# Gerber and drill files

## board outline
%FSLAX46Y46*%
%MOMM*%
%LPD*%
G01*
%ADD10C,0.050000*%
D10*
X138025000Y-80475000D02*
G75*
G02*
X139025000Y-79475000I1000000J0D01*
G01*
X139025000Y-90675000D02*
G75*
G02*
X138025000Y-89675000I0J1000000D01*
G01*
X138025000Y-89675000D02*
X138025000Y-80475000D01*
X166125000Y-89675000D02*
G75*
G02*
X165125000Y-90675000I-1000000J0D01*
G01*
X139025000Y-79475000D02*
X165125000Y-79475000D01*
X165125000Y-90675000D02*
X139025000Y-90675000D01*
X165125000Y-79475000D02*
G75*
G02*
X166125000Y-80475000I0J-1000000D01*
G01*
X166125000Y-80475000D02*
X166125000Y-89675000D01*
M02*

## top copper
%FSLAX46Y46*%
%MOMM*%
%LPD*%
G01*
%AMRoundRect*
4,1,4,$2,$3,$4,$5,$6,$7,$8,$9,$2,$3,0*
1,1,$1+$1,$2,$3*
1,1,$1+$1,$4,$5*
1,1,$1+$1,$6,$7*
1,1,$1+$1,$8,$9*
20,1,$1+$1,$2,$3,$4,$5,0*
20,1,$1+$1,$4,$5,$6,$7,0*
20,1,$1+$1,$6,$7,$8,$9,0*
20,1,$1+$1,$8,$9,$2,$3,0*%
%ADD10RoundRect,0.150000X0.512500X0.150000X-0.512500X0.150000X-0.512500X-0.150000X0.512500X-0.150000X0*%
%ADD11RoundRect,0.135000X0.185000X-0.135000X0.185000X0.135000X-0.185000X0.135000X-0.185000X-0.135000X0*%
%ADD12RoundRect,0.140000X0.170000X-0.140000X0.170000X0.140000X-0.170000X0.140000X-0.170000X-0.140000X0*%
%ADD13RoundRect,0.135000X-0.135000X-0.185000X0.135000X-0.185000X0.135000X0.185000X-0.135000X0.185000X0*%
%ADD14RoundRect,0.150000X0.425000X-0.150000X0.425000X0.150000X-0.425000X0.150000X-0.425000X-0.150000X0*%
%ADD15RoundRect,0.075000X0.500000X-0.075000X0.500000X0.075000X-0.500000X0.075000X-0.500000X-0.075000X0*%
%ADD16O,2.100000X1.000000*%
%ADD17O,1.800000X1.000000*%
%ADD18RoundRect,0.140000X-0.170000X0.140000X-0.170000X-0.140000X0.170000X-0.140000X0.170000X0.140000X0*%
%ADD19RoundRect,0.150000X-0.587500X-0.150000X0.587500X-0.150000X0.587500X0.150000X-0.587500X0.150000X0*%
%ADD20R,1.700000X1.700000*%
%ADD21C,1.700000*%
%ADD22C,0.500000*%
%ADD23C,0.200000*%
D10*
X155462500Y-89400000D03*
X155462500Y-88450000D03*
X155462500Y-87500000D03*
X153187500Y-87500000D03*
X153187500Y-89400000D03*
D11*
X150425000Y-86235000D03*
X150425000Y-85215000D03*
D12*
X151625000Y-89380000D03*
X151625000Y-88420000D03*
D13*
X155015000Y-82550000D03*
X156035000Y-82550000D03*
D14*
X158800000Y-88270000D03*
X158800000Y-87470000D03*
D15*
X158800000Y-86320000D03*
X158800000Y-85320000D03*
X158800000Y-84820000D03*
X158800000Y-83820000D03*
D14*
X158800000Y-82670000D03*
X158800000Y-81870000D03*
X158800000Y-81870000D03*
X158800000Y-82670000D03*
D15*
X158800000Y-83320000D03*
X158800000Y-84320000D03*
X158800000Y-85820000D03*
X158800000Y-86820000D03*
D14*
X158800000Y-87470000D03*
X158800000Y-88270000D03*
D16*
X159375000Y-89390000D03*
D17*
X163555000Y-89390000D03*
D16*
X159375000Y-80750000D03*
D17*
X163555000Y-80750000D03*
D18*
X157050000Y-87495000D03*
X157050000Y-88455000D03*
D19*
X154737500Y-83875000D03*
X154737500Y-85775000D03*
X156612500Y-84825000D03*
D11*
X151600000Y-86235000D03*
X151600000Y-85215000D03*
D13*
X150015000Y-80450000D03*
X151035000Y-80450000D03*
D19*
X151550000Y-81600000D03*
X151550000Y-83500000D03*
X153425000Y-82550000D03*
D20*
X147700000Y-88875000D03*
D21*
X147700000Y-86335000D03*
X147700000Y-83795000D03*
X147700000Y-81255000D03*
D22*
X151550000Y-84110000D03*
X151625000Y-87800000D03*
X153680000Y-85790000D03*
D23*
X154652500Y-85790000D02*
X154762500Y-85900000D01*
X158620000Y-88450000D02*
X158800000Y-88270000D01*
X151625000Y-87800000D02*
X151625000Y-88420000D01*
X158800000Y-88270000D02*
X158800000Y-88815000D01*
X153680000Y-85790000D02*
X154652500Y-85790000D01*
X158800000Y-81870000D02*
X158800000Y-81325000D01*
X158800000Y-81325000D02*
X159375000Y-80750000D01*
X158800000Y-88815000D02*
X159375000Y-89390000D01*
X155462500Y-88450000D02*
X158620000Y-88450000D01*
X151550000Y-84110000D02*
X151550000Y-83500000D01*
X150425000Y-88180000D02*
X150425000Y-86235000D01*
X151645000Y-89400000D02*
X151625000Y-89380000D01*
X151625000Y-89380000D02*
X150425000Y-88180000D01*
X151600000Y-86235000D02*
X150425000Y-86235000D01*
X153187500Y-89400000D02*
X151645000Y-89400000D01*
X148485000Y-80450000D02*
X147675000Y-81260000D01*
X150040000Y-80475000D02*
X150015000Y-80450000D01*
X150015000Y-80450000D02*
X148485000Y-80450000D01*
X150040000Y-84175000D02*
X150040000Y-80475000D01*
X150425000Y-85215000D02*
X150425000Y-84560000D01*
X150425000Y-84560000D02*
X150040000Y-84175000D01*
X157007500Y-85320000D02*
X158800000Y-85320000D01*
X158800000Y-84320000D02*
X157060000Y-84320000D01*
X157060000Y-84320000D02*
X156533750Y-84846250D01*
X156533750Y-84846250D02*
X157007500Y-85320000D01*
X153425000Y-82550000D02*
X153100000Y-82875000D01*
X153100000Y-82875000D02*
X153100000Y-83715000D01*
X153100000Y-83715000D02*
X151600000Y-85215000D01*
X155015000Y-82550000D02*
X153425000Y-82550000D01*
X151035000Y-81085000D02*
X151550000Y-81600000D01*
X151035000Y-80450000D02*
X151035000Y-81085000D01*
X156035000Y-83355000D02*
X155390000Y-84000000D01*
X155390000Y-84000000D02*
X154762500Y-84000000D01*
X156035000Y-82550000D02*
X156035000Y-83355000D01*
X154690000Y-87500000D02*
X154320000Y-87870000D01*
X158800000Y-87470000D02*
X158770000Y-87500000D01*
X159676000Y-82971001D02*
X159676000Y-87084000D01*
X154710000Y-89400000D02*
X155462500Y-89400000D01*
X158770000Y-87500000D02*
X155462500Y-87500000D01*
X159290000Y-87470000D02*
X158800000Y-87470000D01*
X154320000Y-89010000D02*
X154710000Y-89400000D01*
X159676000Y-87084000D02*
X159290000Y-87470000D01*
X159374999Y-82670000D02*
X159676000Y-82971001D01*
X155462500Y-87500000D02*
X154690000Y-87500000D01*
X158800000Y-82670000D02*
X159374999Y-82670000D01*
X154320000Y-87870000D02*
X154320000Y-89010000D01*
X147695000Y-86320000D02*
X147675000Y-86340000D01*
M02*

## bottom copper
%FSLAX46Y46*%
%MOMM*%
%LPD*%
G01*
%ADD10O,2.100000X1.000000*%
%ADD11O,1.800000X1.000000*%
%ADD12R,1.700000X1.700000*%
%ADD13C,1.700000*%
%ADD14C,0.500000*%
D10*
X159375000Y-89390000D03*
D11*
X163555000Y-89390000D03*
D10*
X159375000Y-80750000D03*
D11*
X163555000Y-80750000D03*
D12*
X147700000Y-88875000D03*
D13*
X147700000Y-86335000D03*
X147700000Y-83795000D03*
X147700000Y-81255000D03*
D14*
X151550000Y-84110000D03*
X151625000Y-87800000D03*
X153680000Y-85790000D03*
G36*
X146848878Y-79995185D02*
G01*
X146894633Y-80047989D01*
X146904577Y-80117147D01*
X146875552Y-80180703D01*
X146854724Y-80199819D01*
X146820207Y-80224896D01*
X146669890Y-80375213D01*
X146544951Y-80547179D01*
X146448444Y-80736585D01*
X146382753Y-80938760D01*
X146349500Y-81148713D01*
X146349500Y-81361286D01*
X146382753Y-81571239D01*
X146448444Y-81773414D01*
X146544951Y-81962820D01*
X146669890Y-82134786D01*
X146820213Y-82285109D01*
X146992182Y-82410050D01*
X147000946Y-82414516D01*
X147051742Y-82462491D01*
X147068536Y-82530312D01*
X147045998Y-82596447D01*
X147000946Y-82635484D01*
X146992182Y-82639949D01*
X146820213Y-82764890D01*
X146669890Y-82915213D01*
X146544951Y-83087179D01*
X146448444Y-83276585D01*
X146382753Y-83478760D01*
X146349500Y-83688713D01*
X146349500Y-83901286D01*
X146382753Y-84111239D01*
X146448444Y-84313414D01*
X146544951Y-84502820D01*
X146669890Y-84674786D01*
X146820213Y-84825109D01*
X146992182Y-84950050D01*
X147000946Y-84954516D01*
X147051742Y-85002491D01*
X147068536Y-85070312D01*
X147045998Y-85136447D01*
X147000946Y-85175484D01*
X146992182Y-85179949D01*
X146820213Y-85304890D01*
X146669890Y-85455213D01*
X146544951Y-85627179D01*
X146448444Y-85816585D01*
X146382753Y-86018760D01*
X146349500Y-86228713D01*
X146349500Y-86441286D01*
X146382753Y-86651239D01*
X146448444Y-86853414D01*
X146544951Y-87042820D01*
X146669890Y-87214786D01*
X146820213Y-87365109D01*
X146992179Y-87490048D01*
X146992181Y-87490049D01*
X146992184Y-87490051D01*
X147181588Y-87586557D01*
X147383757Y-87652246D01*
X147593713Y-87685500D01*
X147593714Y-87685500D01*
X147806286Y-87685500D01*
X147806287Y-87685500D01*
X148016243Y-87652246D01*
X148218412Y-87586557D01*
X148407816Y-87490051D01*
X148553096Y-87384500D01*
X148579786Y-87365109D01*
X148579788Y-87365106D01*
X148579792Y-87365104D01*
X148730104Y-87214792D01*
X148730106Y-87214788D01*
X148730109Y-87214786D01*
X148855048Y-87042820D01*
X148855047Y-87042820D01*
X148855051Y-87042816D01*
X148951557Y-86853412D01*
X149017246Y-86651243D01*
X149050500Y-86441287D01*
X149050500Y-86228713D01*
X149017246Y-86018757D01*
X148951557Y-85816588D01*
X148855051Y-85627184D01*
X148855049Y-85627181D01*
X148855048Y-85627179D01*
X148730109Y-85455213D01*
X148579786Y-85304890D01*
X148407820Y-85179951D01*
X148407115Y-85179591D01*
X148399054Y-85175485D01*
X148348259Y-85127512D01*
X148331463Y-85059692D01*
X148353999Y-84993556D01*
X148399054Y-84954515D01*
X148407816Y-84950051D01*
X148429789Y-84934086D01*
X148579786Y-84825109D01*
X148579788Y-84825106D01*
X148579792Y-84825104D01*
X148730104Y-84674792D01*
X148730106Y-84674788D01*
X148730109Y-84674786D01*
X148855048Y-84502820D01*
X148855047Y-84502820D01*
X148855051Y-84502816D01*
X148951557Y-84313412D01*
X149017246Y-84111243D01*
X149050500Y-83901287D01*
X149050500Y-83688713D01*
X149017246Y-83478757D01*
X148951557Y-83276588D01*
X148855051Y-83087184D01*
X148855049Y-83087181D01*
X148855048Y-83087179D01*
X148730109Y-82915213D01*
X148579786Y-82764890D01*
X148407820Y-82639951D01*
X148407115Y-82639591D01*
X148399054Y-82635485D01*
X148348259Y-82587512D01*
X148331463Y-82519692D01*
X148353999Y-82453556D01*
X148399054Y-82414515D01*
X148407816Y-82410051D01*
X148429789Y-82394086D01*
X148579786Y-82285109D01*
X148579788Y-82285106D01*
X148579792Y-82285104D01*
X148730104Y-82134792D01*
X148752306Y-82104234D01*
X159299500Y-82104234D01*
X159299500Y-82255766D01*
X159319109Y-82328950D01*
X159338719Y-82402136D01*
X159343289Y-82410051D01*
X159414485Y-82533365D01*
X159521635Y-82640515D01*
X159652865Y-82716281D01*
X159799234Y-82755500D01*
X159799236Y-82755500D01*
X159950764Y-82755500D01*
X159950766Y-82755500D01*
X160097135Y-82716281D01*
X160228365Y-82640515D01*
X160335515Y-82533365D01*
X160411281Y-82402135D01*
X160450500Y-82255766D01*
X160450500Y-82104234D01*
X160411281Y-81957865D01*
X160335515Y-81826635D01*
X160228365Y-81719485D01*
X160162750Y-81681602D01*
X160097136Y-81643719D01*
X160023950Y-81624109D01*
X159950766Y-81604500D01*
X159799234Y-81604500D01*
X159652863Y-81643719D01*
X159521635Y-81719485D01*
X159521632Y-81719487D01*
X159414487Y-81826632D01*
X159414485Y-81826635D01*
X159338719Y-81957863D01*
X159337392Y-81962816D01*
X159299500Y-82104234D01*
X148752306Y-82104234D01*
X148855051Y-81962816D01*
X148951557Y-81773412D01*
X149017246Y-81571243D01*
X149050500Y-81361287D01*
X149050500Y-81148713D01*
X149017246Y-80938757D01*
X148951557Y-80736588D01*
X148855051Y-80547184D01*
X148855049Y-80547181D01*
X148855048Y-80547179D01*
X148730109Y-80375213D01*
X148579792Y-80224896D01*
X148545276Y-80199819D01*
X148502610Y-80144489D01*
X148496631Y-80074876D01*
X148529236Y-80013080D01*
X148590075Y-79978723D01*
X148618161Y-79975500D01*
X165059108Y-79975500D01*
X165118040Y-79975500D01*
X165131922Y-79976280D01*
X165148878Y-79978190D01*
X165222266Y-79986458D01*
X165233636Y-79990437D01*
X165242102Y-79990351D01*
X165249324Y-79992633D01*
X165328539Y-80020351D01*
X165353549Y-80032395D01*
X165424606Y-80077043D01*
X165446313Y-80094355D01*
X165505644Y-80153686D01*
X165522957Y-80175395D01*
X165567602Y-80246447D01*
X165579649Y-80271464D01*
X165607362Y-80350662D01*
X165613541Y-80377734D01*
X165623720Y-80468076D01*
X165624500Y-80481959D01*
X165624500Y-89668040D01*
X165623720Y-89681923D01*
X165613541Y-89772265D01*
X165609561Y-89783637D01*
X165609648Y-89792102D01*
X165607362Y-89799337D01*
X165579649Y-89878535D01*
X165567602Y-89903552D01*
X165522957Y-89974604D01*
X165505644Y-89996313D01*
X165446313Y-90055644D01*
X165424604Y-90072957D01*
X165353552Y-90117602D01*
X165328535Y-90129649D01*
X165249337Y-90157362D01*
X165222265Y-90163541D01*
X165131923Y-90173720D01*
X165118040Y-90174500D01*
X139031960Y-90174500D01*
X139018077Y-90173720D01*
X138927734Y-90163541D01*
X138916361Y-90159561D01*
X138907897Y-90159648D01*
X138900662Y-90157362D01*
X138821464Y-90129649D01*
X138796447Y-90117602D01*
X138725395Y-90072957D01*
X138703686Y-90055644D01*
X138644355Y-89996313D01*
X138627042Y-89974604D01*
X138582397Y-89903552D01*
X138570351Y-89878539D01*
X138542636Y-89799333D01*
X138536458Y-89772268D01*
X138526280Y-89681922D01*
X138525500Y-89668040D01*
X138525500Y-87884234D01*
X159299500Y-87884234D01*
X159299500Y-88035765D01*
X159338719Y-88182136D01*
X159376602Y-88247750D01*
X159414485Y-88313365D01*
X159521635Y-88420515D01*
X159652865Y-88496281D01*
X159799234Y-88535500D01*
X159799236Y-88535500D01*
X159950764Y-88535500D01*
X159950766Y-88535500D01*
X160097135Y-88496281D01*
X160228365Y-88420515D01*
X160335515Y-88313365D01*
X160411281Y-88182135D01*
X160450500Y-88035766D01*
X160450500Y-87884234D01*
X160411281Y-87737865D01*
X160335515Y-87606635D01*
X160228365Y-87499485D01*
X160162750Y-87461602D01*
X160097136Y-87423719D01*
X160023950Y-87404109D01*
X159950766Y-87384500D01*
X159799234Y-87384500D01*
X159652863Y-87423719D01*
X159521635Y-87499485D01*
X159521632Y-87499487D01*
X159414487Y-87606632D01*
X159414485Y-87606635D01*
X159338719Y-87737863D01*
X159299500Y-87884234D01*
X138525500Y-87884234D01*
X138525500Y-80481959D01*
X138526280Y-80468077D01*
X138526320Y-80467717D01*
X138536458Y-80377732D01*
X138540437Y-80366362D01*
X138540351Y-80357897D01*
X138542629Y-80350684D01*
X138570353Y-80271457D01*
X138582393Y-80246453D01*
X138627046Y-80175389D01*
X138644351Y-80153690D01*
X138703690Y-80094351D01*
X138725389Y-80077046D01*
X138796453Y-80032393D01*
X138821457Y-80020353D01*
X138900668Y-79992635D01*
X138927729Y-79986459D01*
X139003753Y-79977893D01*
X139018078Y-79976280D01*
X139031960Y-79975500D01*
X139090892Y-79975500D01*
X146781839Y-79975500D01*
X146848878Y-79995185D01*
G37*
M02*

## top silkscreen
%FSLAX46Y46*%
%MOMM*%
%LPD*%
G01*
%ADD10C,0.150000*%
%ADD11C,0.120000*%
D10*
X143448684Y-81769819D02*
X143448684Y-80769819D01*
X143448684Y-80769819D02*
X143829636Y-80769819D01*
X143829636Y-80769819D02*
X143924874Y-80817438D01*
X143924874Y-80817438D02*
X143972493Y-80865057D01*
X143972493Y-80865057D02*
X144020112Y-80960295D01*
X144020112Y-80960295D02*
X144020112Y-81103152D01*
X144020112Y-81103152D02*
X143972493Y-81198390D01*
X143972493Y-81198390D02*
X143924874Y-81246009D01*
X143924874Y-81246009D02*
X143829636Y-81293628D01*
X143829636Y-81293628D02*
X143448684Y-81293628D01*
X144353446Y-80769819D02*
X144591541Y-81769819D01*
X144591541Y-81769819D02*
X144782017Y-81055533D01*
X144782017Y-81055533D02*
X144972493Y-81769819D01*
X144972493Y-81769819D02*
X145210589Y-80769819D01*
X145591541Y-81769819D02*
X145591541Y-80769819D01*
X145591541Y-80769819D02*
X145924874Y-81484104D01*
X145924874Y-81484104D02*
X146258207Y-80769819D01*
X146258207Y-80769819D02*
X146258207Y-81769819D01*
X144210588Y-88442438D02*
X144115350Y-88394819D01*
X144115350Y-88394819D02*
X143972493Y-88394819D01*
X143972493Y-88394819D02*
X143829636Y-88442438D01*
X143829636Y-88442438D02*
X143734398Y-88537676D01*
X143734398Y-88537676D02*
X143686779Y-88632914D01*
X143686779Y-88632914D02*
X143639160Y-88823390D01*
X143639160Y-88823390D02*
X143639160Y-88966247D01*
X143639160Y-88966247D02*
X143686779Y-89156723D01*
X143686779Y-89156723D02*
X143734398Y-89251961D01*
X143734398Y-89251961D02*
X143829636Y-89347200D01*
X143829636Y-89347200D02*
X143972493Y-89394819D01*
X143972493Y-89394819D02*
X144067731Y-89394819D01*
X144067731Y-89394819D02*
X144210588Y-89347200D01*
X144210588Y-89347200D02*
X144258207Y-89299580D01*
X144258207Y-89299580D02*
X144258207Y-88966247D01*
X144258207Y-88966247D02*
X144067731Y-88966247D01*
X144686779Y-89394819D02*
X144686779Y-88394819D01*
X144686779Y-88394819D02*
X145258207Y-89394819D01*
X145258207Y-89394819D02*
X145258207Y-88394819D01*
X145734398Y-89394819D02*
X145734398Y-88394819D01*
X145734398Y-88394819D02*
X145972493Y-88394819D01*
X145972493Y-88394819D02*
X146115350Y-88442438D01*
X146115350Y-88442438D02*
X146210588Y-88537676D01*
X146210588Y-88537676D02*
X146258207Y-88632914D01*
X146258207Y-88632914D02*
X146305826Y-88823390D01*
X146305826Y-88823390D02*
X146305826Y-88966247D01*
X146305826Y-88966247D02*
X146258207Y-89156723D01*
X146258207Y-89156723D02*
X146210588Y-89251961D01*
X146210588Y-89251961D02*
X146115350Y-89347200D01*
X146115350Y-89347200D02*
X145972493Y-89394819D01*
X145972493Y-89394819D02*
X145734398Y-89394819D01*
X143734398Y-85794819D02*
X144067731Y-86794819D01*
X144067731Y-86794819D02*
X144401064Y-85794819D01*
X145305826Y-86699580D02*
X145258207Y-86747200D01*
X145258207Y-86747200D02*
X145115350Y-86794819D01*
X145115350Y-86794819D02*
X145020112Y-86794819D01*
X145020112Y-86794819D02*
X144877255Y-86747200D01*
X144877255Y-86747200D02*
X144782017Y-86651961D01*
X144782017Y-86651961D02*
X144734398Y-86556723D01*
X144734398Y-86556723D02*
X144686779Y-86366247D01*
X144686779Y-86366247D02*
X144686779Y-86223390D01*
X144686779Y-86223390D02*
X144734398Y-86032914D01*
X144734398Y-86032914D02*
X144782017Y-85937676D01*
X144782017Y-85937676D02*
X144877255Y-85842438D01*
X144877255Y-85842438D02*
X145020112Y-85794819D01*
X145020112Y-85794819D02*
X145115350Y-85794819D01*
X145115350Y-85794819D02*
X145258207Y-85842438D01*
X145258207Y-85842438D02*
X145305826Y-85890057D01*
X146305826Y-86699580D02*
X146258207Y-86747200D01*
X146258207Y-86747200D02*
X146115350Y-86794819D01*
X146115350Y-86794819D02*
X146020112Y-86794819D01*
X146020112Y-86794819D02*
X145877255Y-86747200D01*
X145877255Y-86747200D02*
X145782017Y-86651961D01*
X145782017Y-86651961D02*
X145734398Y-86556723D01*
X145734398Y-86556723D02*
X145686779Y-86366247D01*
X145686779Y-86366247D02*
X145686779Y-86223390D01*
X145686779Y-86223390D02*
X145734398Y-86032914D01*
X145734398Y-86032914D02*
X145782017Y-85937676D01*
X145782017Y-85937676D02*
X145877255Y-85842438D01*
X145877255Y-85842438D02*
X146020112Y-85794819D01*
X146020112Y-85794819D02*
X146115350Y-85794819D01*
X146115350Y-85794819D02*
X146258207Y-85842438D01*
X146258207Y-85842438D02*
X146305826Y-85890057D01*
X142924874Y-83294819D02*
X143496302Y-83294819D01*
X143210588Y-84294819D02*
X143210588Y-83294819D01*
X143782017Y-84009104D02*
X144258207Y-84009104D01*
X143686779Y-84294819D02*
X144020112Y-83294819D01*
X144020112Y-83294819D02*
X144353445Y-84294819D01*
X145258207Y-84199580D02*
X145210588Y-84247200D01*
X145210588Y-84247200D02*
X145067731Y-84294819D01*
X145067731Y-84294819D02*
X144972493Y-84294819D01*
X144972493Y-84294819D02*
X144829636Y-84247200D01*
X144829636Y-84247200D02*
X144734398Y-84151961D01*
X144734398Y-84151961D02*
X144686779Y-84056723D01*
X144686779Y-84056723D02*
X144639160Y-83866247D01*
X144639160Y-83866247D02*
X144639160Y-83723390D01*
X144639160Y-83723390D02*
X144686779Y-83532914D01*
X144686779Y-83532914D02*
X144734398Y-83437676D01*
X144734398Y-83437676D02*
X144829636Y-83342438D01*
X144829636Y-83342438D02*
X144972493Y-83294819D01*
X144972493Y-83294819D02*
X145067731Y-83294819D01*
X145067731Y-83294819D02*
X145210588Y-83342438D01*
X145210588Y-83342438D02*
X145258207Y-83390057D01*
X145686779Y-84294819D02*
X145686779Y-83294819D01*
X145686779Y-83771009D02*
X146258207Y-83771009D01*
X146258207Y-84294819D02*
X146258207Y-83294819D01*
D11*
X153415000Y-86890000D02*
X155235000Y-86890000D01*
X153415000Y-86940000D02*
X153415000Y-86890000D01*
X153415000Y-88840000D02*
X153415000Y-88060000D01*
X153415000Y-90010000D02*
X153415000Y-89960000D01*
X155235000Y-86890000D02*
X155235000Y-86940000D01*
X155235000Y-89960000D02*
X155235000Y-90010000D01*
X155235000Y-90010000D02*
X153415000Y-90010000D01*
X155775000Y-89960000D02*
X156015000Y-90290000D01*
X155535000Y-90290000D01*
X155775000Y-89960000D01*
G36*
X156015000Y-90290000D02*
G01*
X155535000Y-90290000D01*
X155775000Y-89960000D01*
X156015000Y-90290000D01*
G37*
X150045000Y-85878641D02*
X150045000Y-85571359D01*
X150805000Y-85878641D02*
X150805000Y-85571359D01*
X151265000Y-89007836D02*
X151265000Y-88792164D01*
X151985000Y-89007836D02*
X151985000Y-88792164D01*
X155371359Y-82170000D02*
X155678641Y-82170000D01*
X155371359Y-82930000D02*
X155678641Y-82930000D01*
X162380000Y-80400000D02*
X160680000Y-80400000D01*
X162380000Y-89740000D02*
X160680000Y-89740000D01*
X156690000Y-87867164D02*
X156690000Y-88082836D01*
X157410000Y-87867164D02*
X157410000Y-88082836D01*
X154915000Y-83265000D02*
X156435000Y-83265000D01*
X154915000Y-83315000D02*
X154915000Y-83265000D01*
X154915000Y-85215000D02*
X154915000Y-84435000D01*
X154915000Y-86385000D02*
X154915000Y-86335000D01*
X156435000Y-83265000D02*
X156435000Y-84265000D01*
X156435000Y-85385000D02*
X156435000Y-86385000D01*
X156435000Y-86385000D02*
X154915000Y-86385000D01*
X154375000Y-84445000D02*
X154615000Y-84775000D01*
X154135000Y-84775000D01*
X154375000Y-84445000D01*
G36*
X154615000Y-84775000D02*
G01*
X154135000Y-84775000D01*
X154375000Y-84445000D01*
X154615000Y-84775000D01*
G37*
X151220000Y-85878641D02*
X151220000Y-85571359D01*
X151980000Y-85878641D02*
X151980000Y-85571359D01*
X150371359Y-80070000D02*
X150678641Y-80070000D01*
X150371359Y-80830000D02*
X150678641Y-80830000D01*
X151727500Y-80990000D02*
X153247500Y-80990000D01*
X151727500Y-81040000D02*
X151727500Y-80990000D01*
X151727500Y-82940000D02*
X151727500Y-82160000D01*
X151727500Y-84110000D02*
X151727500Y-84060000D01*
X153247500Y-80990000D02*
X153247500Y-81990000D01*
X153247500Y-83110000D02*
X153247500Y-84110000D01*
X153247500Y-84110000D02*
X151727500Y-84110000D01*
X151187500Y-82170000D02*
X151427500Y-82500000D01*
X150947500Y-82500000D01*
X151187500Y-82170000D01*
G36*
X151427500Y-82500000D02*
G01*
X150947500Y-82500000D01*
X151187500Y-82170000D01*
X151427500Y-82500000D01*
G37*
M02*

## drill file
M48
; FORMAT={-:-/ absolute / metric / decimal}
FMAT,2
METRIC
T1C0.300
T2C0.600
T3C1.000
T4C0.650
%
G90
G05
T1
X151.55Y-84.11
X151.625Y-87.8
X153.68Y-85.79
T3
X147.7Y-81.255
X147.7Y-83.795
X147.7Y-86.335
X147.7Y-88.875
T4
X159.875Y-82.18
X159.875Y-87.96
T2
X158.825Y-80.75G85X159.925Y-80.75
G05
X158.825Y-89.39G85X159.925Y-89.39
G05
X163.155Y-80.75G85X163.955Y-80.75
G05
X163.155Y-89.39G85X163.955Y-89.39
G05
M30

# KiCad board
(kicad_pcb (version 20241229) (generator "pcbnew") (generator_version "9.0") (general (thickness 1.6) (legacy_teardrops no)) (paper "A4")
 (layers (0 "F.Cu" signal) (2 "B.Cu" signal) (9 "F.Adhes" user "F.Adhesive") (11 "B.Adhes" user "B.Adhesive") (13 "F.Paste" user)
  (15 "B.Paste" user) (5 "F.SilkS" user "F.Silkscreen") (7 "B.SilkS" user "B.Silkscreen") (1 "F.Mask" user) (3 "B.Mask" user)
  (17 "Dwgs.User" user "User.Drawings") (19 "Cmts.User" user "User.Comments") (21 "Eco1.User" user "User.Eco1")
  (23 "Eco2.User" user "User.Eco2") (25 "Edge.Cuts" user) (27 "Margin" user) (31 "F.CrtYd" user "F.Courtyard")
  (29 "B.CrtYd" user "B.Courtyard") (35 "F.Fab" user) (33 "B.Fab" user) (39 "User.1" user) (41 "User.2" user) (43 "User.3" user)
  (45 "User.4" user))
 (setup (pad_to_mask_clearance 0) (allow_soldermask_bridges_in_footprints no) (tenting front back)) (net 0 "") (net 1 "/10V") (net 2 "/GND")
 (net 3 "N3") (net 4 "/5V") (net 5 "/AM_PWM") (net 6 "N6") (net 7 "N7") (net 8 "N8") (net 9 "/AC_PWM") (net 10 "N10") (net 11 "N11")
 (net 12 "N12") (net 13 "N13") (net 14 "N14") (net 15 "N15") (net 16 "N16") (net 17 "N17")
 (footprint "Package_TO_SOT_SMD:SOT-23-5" (layer "F.Cu") (at 154.325 88.45 180)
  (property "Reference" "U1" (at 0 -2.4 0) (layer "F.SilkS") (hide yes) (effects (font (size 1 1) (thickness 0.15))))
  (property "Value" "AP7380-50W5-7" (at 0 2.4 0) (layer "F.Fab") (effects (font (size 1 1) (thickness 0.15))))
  (fp_line (start 0.91 1.56) (end -0.91 1.56) (stroke (width 0.12) (type solid)) (layer "F.SilkS"))
  (fp_line (start 0.91 1.51) (end 0.91 1.56) (stroke (width 0.12) (type solid)) (layer "F.SilkS"))
  (fp_line (start 0.91 -0.39) (end 0.91 0.39) (stroke (width 0.12) (type solid)) (layer "F.SilkS"))
  (fp_line (start 0.91 -1.56) (end 0.91 -1.51) (stroke (width 0.12) (type solid)) (layer "F.SilkS"))
  (fp_line (start -0.91 1.56) (end -0.91 1.51) (stroke (width 0.12) (type solid)) (layer "F.SilkS"))
  (fp_line (start -0.91 -1.51) (end -0.91 -1.56) (stroke (width 0.12) (type solid)) (layer "F.SilkS"))
  (fp_line (start -0.91 -1.56) (end 0.91 -1.56) (stroke (width 0.12) (type solid)) (layer "F.SilkS"))
  (fp_poly (pts (xy -1.45 -1.51) (xy -1.69 -1.84) (xy -1.21 -1.84)) (stroke (width 0.12) (type solid)) (fill yes) (layer "F.SilkS"))
  (pad "1" smd roundrect (at -1.1375 -0.95 180) (size 1.325 0.6) (layers "F.Cu" "F.Mask" "F.Paste") (roundrect_rratio 0.25) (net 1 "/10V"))
  (pad "2" smd roundrect (at -1.1375 0 180) (size 1.325 0.6) (layers "F.Cu" "F.Mask" "F.Paste") (roundrect_rratio 0.25) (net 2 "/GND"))
  (pad "3" smd roundrect (at -1.1375 0.95 180) (size 1.325 0.6) (layers "F.Cu" "F.Mask" "F.Paste") (roundrect_rratio 0.25) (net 1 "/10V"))
  (pad "4" smd roundrect (at 1.1375 0.95 180) (size 1.325 0.6) (layers "F.Cu" "F.Mask" "F.Paste") (roundrect_rratio 0.25) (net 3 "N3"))
  (pad "5" smd roundrect (at 1.1375 -0.95 180) (size 1.325 0.6) (layers "F.Cu" "F.Mask" "F.Paste") (roundrect_rratio 0.25) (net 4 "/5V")))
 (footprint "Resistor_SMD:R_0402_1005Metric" (layer "F.Cu") (at 150.425 85.725 90)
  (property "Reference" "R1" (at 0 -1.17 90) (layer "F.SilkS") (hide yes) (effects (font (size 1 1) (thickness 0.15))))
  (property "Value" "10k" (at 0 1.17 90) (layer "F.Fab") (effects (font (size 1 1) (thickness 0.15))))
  (fp_line (start -0.153641 -0.38) (end 0.153641 -0.38) (stroke (width 0.12) (type solid)) (layer "F.SilkS"))
  (fp_line (start -0.153641 0.38) (end 0.153641 0.38) (stroke (width 0.12) (type solid)) (layer "F.SilkS"))
  (pad "1" smd roundrect (at -0.51 0 90) (size 0.54 0.64) (layers "F.Cu" "F.Mask" "F.Paste") (roundrect_rratio 0.25) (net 4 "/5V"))
  (pad "2" smd roundrect (at 0.51 0 90) (size 0.54 0.64) (layers "F.Cu" "F.Mask" "F.Paste") (roundrect_rratio 0.25) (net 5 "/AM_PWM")))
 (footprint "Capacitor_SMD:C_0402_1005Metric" (layer "F.Cu") (at 151.625 88.9 90)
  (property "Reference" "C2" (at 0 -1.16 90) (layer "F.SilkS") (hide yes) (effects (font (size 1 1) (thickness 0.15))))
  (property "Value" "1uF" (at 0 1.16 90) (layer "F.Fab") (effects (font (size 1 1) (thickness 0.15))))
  (fp_line (start -0.107836 -0.36) (end 0.107836 -0.36) (stroke (width 0.12) (type solid)) (layer "F.SilkS"))
  (fp_line (start -0.107836 0.36) (end 0.107836 0.36) (stroke (width 0.12) (type solid)) (layer "F.SilkS"))
  (pad "1" smd roundrect (at -0.48 0 90) (size 0.56 0.62) (layers "F.Cu" "F.Mask" "F.Paste") (roundrect_rratio 0.25) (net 4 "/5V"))
  (pad "2" smd roundrect (at 0.48 0 90) (size 0.56 0.62) (layers "F.Cu" "F.Mask" "F.Paste") (roundrect_rratio 0.25) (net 2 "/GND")))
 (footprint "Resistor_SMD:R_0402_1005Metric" (layer "F.Cu") (at 155.525 82.55)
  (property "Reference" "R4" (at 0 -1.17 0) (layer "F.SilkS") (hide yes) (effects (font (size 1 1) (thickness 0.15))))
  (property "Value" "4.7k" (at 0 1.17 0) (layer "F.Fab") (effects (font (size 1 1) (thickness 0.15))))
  (fp_line (start -0.153641 -0.38) (end 0.153641 -0.38) (stroke (width 0.12) (type solid)) (layer "F.SilkS"))
  (fp_line (start -0.153641 0.38) (end 0.153641 0.38) (stroke (width 0.12) (type solid)) (layer "F.SilkS"))
  (pad "1" smd roundrect (at -0.51 0) (size 0.54 0.64) (layers "F.Cu" "F.Mask" "F.Paste") (roundrect_rratio 0.25) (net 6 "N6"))
  (pad "2" smd roundrect (at 0.51 0) (size 0.54 0.64) (layers "F.Cu" "F.Mask" "F.Paste") (roundrect_rratio 0.25) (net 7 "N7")))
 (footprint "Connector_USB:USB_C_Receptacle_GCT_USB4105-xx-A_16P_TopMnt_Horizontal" (layer "F.Cu") (at 162.48 85.07 90)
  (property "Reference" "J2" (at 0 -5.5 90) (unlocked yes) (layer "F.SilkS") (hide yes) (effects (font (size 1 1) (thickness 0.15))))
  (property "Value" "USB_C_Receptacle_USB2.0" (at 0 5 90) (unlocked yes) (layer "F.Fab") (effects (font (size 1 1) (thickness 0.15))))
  (fp_line (start 4.67 -0.1) (end 4.67 -1.8) (stroke (width 0.12) (type solid)) (layer "F.SilkS"))
  (fp_line (start -4.67 -0.1) (end -4.67 -1.8) (stroke (width 0.12) (type solid)) (layer "F.SilkS"))
  (pad "" np_thru_hole circle (at -2.89 -2.605 90) (size 0.65 0.65) (drill 0.65) (layers "*.Cu" "*.Mask"))
  (pad "" np_thru_hole circle (at 2.89 -2.605 90) (size 0.65 0.65) (drill 0.65) (layers "*.Cu" "*.Mask"))
  (pad "A1" smd roundrect (at -3.2 -3.68 90) (size 0.6 1.15) (layers "F.Cu" "F.Mask" "F.Paste") (roundrect_rratio 0.25) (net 2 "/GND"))
  (pad "A4" smd roundrect (at -2.4 -3.68 90) (size 0.6 1.15) (layers "F.Cu" "F.Mask" "F.Paste") (roundrect_rratio 0.25) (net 1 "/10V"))
  (pad "A5" smd roundrect (at -1.25 -3.68 90) (size 0.3 1.15) (layers "F.Cu" "F.Mask" "F.Paste") (roundrect_rratio 0.25) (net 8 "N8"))
  (pad "A6" smd roundrect (at -0.25 -3.68 90) (size 0.3 1.15) (layers "F.Cu" "F.Mask" "F.Paste") (roundrect_rratio 0.25) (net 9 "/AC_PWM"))
  (pad "A7" smd roundrect (at 0.25 -3.68 90) (size 0.3 1.15) (layers "F.Cu" "F.Mask" "F.Paste") (roundrect_rratio 0.25) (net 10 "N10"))
  (pad "A8" smd roundrect (at 1.25 -3.68 90) (size 0.3 1.15) (layers "F.Cu" "F.Mask" "F.Paste") (roundrect_rratio 0.25) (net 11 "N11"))
  (pad "A9" smd roundrect (at 2.4 -3.68 90) (size 0.6 1.15) (layers "F.Cu" "F.Mask" "F.Paste") (roundrect_rratio 0.25) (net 1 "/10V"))
  (pad "A12" smd roundrect (at 3.2 -3.68 90) (size 0.6 1.15) (layers "F.Cu" "F.Mask" "F.Paste") (roundrect_rratio 0.25) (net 2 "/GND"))
  (pad "B1" smd roundrect (at 3.2 -3.68 90) (size 0.6 1.15) (layers "F.Cu" "F.Mask" "F.Paste") (roundrect_rratio 0.25) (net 2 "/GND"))
  (pad "B4" smd roundrect (at 2.4 -3.68 90) (size 0.6 1.15) (layers "F.Cu" "F.Mask" "F.Paste") (roundrect_rratio 0.25) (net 1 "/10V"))
  (pad "B5" smd roundrect (at 1.75 -3.68 90) (size 0.3 1.15) (layers "F.Cu" "F.Mask" "F.Paste") (roundrect_rratio 0.25) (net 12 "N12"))
  (pad "B6" smd roundrect (at 0.75 -3.68 90) (size 0.3 1.15) (layers "F.Cu" "F.Mask" "F.Paste") (roundrect_rratio 0.25) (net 9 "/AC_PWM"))
  (pad "B7" smd roundrect (at -0.75 -3.68 90) (size 0.3 1.15) (layers "F.Cu" "F.Mask" "F.Paste") (roundrect_rratio 0.25) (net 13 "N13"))
  (pad "B8" smd roundrect (at -1.75 -3.68 90) (size 0.3 1.15) (layers "F.Cu" "F.Mask" "F.Paste") (roundrect_rratio 0.25) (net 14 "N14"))
  (pad "B9" smd roundrect (at -2.4 -3.68 90) (size 0.6 1.15) (layers "F.Cu" "F.Mask" "F.Paste") (roundrect_rratio 0.25) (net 1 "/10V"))
  (pad "B12" smd roundrect (at -3.2 -3.68 90) (size 0.6 1.15) (layers "F.Cu" "F.Mask" "F.Paste") (roundrect_rratio 0.25) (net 2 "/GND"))
  (pad "S1" thru_hole oval (at -4.32 -3.105 90) (size 1 2.1) (drill oval 0.6 1.7) (layers "*.Cu" "*.Mask" "F.Paste")
   (remove_unused_layers no) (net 2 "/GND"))
  (pad "S1" thru_hole oval (at -4.32 1.075 90) (size 1 1.8) (drill oval 0.6 1.4) (layers "*.Cu" "*.Mask" "F.Paste")
   (remove_unused_layers no) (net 2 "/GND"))
  (pad "S1" thru_hole oval (at 4.32 -3.105 90) (size 1 2.1) (drill oval 0.6 1.7) (layers "*.Cu" "*.Mask" "F.Paste")
   (remove_unused_layers yes) (keep_end_layers yes) (zone_layer_connections) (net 2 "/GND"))
  (pad "S1" thru_hole oval (at 4.32 1.075 90) (size 1 1.8) (drill oval 0.6 1.4) (layers "*.Cu" "*.Mask" "F.Paste") (remove_unused_layers no)
   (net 2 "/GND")))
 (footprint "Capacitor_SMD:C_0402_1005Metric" (layer "F.Cu") (at 157.05 87.975 -90)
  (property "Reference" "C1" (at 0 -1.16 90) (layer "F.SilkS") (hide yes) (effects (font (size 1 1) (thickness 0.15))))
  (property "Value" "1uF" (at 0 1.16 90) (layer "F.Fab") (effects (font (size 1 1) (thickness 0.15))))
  (fp_line (start -0.107836 0.36) (end 0.107836 0.36) (stroke (width 0.12) (type solid)) (layer "F.SilkS"))
  (fp_line (start -0.107836 -0.36) (end 0.107836 -0.36) (stroke (width 0.12) (type solid)) (layer "F.SilkS"))
  (pad "1" smd roundrect (at -0.48 0 270) (size 0.56 0.62) (layers "F.Cu" "F.Mask" "F.Paste") (roundrect_rratio 0.25) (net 1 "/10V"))
  (pad "2" smd roundrect (at 0.48 0 270) (size 0.56 0.62) (layers "F.Cu" "F.Mask" "F.Paste") (roundrect_rratio 0.25) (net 2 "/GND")))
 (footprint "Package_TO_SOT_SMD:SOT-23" (layer "F.Cu") (at 155.675 84.825)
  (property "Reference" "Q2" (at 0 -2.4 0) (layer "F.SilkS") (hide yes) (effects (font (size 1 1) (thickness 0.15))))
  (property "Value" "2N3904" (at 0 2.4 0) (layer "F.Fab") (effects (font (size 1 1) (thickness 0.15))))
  (fp_line (start -0.76 -1.56) (end 0.76 -1.56) (stroke (width 0.12) (type solid)) (layer "F.SilkS"))
  (fp_line (start -0.76 -1.51) (end -0.76 -1.56) (stroke (width 0.12) (type solid)) (layer "F.SilkS"))
  (fp_line (start -0.76 0.39) (end -0.76 -0.39) (stroke (width 0.12) (type solid)) (layer "F.SilkS"))
  (fp_line (start -0.76 1.56) (end -0.76 1.51) (stroke (width 0.12) (type solid)) (layer "F.SilkS"))
  (fp_line (start 0.76 -1.56) (end 0.76 -0.56) (stroke (width 0.12) (type solid)) (layer "F.SilkS"))
  (fp_line (start 0.76 0.56) (end 0.76 1.56) (stroke (width 0.12) (type solid)) (layer "F.SilkS"))
  (fp_line (start 0.76 1.56) (end -0.76 1.56) (stroke (width 0.12) (type solid)) (layer "F.SilkS"))
  (fp_poly (pts (xy -1.3 -0.38) (xy -1.06 -0.05) (xy -1.54 -0.05)) (stroke (width 0.12) (type solid)) (fill yes) (layer "F.SilkS"))
  (pad "1" smd roundrect (at -0.9375 -0.95) (size 1.475 0.6) (layers "F.Cu" "F.Mask" "F.Paste") (roundrect_rratio 0.25) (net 7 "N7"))
  (pad "2" smd roundrect (at -0.9375 0.95) (size 1.475 0.6) (layers "F.Cu" "F.Mask" "F.Paste") (roundrect_rratio 0.25) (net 2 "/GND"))
  (pad "3" smd roundrect (at 0.9375 0) (size 1.475 0.6) (layers "F.Cu" "F.Mask" "F.Paste") (roundrect_rratio 0.25) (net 9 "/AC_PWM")))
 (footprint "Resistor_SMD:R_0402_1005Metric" (layer "F.Cu") (at 151.6 85.725 90)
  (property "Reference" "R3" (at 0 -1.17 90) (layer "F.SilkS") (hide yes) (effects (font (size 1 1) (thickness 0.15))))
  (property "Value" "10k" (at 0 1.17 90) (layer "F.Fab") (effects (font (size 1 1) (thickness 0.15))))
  (fp_line (start -0.153641 -0.38) (end 0.153641 -0.38) (stroke (width 0.12) (type solid)) (layer "F.SilkS"))
  (fp_line (start -0.153641 0.38) (end 0.153641 0.38) (stroke (width 0.12) (type solid)) (layer "F.SilkS"))
  (pad "1" smd roundrect (at -0.51 0 90) (size 0.54 0.64) (layers "F.Cu" "F.Mask" "F.Paste") (roundrect_rratio 0.25) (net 4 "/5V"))
  (pad "2" smd roundrect (at 0.51 0 90) (size 0.54 0.64) (layers "F.Cu" "F.Mask" "F.Paste") (roundrect_rratio 0.25) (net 6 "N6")))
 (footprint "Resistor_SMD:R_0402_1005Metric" (layer "F.Cu") (at 150.525 80.45)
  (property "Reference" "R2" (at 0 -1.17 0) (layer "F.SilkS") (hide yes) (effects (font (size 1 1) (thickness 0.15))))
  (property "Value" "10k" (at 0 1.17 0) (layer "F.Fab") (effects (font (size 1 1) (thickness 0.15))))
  (fp_line (start -0.153641 -0.38) (end 0.153641 -0.38) (stroke (width 0.12) (type solid)) (layer "F.SilkS"))
  (fp_line (start -0.153641 0.38) (end 0.153641 0.38) (stroke (width 0.12) (type solid)) (layer "F.SilkS"))
  (pad "1" smd roundrect (at -0.51 0) (size 0.54 0.64) (layers "F.Cu" "F.Mask" "F.Paste") (roundrect_rratio 0.25) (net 5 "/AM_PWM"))
  (pad "2" smd roundrect (at 0.51 0) (size 0.54 0.64) (layers "F.Cu" "F.Mask" "F.Paste") (roundrect_rratio 0.25) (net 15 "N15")))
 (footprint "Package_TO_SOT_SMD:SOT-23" (layer "F.Cu") (at 152.4875 82.55)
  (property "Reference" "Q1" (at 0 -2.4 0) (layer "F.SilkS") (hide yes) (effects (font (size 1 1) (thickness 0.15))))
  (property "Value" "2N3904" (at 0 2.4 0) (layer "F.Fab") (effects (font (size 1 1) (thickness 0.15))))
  (fp_line (start -0.76 -1.56) (end 0.76 -1.56) (stroke (width 0.12) (type solid)) (layer "F.SilkS"))
  (fp_line (start -0.76 -1.51) (end -0.76 -1.56) (stroke (width 0.12) (type solid)) (layer "F.SilkS"))
  (fp_line (start -0.76 0.39) (end -0.76 -0.39) (stroke (width 0.12) (type solid)) (layer "F.SilkS"))
  (fp_line (start -0.76 1.56) (end -0.76 1.51) (stroke (width 0.12) (type solid)) (layer "F.SilkS"))
  (fp_line (start 0.76 -1.56) (end 0.76 -0.56) (stroke (width 0.12) (type solid)) (layer "F.SilkS"))
  (fp_line (start 0.76 0.56) (end 0.76 1.56) (stroke (width 0.12) (type solid)) (layer "F.SilkS"))
  (fp_line (start 0.76 1.56) (end -0.76 1.56) (stroke (width 0.12) (type solid)) (layer "F.SilkS"))
  (fp_poly (pts (xy -1.3 -0.38) (xy -1.06 -0.05) (xy -1.54 -0.05)) (stroke (width 0.12) (type solid)) (fill yes) (layer "F.SilkS"))
  (pad "1" smd roundrect (at -0.9375 -0.95) (size 1.475 0.6) (layers "F.Cu" "F.Mask" "F.Paste") (roundrect_rratio 0.25) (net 15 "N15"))
  (pad "2" smd roundrect (at -0.9375 0.95) (size 1.475 0.6) (layers "F.Cu" "F.Mask" "F.Paste") (roundrect_rratio 0.25) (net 2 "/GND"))
  (pad "3" smd roundrect (at 0.9375 0) (size 1.475 0.6) (layers "F.Cu" "F.Mask" "F.Paste") (roundrect_rratio 0.25) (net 6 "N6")))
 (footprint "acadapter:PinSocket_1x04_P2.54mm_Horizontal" (layer "B.Cu") (at 147.7 88.875)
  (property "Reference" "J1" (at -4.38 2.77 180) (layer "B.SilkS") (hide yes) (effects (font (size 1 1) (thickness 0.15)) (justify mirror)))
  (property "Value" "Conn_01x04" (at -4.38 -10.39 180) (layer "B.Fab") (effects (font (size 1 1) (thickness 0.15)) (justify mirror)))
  (pad "1" thru_hole rect (at 0 0) (size 1.7 1.7) (drill 1) (layers "*.Cu" "*.Mask") (remove_unused_layers no) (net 2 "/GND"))
  (pad "2" thru_hole circle (at 0 -2.54) (size 1.7 1.7) (drill 1) (layers "*.Cu" "*.Mask") (remove_unused_layers no) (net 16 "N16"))
  (pad "3" thru_hole circle (at 0 -5.08) (size 1.7 1.7) (drill 1) (layers "*.Cu" "*.Mask") (remove_unused_layers no) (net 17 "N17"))
  (pad "4" thru_hole circle (at 0 -7.62) (size 1.7 1.7) (drill 1) (layers "*.Cu" "*.Mask") (remove_unused_layers no) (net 5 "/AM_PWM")))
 (gr_arc (start 138.025 80.475) (mid 138.317893 79.767893) (end 139.025 79.475) (stroke (width 0.05) (type default)) (layer "Edge.Cuts"))
 (gr_arc (start 139.025 90.675) (mid 138.317893 90.382107) (end 138.025 89.675) (stroke (width 0.05) (type default)) (layer "Edge.Cuts"))
 (gr_line (start 138.025 89.675) (end 138.025 80.475) (stroke (width 0.05) (type default)) (layer "Edge.Cuts"))
 (gr_arc (start 166.125 89.675) (mid 165.832107 90.382107) (end 165.125 90.675) (stroke (width 0.05) (type default)) (layer "Edge.Cuts"))
 (gr_line (start 139.025 79.475) (end 165.125 79.475) (stroke (width 0.05) (type default)) (layer "Edge.Cuts"))
 (gr_line (start 165.125 90.675) (end 139.025 90.675) (stroke (width 0.05) (type default)) (layer "Edge.Cuts"))
 (gr_arc (start 165.125 79.475) (mid 165.832107 79.767893) (end 166.125 80.475) (stroke (width 0.05) (type default)) (layer "Edge.Cuts"))
 (gr_line (start 166.125 80.475) (end 166.125 89.675) (stroke (width 0.05) (type default)) (layer "Edge.Cuts"))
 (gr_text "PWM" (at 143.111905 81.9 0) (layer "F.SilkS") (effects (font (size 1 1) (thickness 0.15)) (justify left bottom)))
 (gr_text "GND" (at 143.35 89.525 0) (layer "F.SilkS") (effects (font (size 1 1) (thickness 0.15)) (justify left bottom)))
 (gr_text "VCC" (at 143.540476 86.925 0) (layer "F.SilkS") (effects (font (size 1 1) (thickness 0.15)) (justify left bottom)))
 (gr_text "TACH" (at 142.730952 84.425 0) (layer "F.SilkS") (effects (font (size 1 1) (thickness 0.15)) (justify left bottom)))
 (segment (start 154.6525 85.79) (end 154.7625 85.9) (width 0.2) (layer "F.Cu") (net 2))
 (segment (start 158.62 88.45) (end 158.8 88.27) (width 0.2) (layer "F.Cu") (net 2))
 (segment (start 151.625 87.8) (end 151.625 88.42) (width 0.2) (layer "F.Cu") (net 2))
 (segment (start 158.8 88.27) (end 158.8 88.815) (width 0.2) (layer "F.Cu") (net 2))
 (segment (start 153.68 85.79) (end 154.6525 85.79) (width 0.2) (layer "F.Cu") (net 2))
 (segment (start 158.8 81.87) (end 158.8 81.325) (width 0.2) (layer "F.Cu") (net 2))
 (segment (start 158.8 81.325) (end 159.375 80.75) (width 0.2) (layer "F.Cu") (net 2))
 (segment (start 158.8 88.815) (end 159.375 89.39) (width 0.2) (layer "F.Cu") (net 2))
 (segment (start 155.4625 88.45) (end 158.62 88.45) (width 0.2) (layer "F.Cu") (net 2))
 (segment (start 151.55 84.11) (end 151.55 83.5) (width 0.2) (layer "F.Cu") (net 2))
 (via (at 151.55 84.11) (size 0.5) (drill 0.3) (layers "F.Cu" "B.Cu") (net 2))
 (via (at 151.625 87.8) (size 0.5) (drill 0.3) (layers "F.Cu" "B.Cu") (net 2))
 (via (at 153.68 85.79) (size 0.5) (drill 0.3) (layers "F.Cu" "B.Cu") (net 2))
 (segment (start 150.425 88.18) (end 150.425 86.235) (width 0.2) (layer "F.Cu") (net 4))
 (segment (start 151.645 89.4) (end 151.625 89.38) (width 0.2) (layer "F.Cu") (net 4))
 (segment (start 151.625 89.38) (end 150.425 88.18) (width 0.2) (layer "F.Cu") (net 4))
 (segment (start 151.6 86.235) (end 150.425 86.235) (width 0.2) (layer "F.Cu") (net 4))
 (segment (start 153.1875 89.4) (end 151.645 89.4) (width 0.2) (layer "F.Cu") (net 4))
 (segment (start 148.485 80.45) (end 147.675 81.26) (width 0.2) (layer "F.Cu") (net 5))
 (segment (start 150.04 80.475) (end 150.015 80.45) (width 0.2) (layer "F.Cu") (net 5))
 (segment (start 150.015 80.45) (end 148.485 80.45) (width 0.2) (layer "F.Cu") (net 5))
 (segment (start 150.04 84.175) (end 150.04 80.475) (width 0.2) (layer "F.Cu") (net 5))
 (segment (start 150.425 85.215) (end 150.425 84.56) (width 0.2) (layer "F.Cu") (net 5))
 (segment (start 150.425 84.56) (end 150.04 84.175) (width 0.2) (layer "F.Cu") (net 5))
 (segment (start 157.0075 85.32) (end 158.8 85.32) (width 0.2) (layer "F.Cu") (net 9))
 (segment (start 158.8 84.32) (end 157.06 84.32) (width 0.2) (layer "F.Cu") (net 9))
 (segment (start 157.06 84.32) (end 156.53375 84.84625) (width 0.2) (layer "F.Cu") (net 9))
 (segment (start 156.53375 84.84625) (end 157.0075 85.32) (width 0.2) (layer "F.Cu") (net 9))
 (segment (start 153.425 82.55) (end 153.1 82.875) (width 0.2) (layer "F.Cu") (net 6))
 (segment (start 153.1 82.875) (end 153.1 83.715) (width 0.2) (layer "F.Cu") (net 6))
 (segment (start 153.1 83.715) (end 151.6 85.215) (width 0.2) (layer "F.Cu") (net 6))
 (segment (start 155.015 82.55) (end 153.425 82.55) (width 0.2) (layer "F.Cu") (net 6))
 (segment (start 151.035 81.085) (end 151.55 81.6) (width 0.2) (layer "F.Cu") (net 15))
 (segment (start 151.035 80.45) (end 151.035 81.085) (width 0.2) (layer "F.Cu") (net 15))
 (segment (start 156.035 83.355) (end 155.39 84) (width 0.2) (layer "F.Cu") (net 7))
 (segment (start 155.39 84) (end 154.7625 84) (width 0.2) (layer "F.Cu") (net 7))
 (segment (start 156.035 82.55) (end 156.035 83.355) (width 0.2) (layer "F.Cu") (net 7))
 (segment (start 154.69 87.5) (end 154.32 87.87) (width 0.2) (layer "F.Cu") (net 1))
 (segment (start 158.8 87.47) (end 158.77 87.5) (width 0.2) (layer "F.Cu") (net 1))
 (segment (start 159.676 82.971001) (end 159.676 87.084) (width 0.2) (layer "F.Cu") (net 1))
 (segment (start 154.71 89.4) (end 155.4625 89.4) (width 0.2) (layer "F.Cu") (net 1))
 (segment (start 158.77 87.5) (end 155.4625 87.5) (width 0.2) (layer "F.Cu") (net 1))
 (segment (start 159.29 87.47) (end 158.8 87.47) (width 0.2) (layer "F.Cu") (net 1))
 (segment (start 154.32 89.01) (end 154.71 89.4) (width 0.2) (layer "F.Cu") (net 1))
 (segment (start 159.676 87.084) (end 159.29 87.47) (width 0.2) (layer "F.Cu") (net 1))
 (segment (start 159.374999 82.67) (end 159.676 82.971001) (width 0.2) (layer "F.Cu") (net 1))
 (segment (start 155.4625 87.5) (end 154.69 87.5) (width 0.2) (layer "F.Cu") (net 1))
 (segment (start 158.8 82.67) (end 159.374999 82.67) (width 0.2) (layer "F.Cu") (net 1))
 (segment (start 154.32 87.87) (end 154.32 89.01) (width 0.2) (layer "F.Cu") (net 1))
 (segment (start 147.695 86.32) (end 147.675 86.34) (width 0.2) (layer "F.Cu") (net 16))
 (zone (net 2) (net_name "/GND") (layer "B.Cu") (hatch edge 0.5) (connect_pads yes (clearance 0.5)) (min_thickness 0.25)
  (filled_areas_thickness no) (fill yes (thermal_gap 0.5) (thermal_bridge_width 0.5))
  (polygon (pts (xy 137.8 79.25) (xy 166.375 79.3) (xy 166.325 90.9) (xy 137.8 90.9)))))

